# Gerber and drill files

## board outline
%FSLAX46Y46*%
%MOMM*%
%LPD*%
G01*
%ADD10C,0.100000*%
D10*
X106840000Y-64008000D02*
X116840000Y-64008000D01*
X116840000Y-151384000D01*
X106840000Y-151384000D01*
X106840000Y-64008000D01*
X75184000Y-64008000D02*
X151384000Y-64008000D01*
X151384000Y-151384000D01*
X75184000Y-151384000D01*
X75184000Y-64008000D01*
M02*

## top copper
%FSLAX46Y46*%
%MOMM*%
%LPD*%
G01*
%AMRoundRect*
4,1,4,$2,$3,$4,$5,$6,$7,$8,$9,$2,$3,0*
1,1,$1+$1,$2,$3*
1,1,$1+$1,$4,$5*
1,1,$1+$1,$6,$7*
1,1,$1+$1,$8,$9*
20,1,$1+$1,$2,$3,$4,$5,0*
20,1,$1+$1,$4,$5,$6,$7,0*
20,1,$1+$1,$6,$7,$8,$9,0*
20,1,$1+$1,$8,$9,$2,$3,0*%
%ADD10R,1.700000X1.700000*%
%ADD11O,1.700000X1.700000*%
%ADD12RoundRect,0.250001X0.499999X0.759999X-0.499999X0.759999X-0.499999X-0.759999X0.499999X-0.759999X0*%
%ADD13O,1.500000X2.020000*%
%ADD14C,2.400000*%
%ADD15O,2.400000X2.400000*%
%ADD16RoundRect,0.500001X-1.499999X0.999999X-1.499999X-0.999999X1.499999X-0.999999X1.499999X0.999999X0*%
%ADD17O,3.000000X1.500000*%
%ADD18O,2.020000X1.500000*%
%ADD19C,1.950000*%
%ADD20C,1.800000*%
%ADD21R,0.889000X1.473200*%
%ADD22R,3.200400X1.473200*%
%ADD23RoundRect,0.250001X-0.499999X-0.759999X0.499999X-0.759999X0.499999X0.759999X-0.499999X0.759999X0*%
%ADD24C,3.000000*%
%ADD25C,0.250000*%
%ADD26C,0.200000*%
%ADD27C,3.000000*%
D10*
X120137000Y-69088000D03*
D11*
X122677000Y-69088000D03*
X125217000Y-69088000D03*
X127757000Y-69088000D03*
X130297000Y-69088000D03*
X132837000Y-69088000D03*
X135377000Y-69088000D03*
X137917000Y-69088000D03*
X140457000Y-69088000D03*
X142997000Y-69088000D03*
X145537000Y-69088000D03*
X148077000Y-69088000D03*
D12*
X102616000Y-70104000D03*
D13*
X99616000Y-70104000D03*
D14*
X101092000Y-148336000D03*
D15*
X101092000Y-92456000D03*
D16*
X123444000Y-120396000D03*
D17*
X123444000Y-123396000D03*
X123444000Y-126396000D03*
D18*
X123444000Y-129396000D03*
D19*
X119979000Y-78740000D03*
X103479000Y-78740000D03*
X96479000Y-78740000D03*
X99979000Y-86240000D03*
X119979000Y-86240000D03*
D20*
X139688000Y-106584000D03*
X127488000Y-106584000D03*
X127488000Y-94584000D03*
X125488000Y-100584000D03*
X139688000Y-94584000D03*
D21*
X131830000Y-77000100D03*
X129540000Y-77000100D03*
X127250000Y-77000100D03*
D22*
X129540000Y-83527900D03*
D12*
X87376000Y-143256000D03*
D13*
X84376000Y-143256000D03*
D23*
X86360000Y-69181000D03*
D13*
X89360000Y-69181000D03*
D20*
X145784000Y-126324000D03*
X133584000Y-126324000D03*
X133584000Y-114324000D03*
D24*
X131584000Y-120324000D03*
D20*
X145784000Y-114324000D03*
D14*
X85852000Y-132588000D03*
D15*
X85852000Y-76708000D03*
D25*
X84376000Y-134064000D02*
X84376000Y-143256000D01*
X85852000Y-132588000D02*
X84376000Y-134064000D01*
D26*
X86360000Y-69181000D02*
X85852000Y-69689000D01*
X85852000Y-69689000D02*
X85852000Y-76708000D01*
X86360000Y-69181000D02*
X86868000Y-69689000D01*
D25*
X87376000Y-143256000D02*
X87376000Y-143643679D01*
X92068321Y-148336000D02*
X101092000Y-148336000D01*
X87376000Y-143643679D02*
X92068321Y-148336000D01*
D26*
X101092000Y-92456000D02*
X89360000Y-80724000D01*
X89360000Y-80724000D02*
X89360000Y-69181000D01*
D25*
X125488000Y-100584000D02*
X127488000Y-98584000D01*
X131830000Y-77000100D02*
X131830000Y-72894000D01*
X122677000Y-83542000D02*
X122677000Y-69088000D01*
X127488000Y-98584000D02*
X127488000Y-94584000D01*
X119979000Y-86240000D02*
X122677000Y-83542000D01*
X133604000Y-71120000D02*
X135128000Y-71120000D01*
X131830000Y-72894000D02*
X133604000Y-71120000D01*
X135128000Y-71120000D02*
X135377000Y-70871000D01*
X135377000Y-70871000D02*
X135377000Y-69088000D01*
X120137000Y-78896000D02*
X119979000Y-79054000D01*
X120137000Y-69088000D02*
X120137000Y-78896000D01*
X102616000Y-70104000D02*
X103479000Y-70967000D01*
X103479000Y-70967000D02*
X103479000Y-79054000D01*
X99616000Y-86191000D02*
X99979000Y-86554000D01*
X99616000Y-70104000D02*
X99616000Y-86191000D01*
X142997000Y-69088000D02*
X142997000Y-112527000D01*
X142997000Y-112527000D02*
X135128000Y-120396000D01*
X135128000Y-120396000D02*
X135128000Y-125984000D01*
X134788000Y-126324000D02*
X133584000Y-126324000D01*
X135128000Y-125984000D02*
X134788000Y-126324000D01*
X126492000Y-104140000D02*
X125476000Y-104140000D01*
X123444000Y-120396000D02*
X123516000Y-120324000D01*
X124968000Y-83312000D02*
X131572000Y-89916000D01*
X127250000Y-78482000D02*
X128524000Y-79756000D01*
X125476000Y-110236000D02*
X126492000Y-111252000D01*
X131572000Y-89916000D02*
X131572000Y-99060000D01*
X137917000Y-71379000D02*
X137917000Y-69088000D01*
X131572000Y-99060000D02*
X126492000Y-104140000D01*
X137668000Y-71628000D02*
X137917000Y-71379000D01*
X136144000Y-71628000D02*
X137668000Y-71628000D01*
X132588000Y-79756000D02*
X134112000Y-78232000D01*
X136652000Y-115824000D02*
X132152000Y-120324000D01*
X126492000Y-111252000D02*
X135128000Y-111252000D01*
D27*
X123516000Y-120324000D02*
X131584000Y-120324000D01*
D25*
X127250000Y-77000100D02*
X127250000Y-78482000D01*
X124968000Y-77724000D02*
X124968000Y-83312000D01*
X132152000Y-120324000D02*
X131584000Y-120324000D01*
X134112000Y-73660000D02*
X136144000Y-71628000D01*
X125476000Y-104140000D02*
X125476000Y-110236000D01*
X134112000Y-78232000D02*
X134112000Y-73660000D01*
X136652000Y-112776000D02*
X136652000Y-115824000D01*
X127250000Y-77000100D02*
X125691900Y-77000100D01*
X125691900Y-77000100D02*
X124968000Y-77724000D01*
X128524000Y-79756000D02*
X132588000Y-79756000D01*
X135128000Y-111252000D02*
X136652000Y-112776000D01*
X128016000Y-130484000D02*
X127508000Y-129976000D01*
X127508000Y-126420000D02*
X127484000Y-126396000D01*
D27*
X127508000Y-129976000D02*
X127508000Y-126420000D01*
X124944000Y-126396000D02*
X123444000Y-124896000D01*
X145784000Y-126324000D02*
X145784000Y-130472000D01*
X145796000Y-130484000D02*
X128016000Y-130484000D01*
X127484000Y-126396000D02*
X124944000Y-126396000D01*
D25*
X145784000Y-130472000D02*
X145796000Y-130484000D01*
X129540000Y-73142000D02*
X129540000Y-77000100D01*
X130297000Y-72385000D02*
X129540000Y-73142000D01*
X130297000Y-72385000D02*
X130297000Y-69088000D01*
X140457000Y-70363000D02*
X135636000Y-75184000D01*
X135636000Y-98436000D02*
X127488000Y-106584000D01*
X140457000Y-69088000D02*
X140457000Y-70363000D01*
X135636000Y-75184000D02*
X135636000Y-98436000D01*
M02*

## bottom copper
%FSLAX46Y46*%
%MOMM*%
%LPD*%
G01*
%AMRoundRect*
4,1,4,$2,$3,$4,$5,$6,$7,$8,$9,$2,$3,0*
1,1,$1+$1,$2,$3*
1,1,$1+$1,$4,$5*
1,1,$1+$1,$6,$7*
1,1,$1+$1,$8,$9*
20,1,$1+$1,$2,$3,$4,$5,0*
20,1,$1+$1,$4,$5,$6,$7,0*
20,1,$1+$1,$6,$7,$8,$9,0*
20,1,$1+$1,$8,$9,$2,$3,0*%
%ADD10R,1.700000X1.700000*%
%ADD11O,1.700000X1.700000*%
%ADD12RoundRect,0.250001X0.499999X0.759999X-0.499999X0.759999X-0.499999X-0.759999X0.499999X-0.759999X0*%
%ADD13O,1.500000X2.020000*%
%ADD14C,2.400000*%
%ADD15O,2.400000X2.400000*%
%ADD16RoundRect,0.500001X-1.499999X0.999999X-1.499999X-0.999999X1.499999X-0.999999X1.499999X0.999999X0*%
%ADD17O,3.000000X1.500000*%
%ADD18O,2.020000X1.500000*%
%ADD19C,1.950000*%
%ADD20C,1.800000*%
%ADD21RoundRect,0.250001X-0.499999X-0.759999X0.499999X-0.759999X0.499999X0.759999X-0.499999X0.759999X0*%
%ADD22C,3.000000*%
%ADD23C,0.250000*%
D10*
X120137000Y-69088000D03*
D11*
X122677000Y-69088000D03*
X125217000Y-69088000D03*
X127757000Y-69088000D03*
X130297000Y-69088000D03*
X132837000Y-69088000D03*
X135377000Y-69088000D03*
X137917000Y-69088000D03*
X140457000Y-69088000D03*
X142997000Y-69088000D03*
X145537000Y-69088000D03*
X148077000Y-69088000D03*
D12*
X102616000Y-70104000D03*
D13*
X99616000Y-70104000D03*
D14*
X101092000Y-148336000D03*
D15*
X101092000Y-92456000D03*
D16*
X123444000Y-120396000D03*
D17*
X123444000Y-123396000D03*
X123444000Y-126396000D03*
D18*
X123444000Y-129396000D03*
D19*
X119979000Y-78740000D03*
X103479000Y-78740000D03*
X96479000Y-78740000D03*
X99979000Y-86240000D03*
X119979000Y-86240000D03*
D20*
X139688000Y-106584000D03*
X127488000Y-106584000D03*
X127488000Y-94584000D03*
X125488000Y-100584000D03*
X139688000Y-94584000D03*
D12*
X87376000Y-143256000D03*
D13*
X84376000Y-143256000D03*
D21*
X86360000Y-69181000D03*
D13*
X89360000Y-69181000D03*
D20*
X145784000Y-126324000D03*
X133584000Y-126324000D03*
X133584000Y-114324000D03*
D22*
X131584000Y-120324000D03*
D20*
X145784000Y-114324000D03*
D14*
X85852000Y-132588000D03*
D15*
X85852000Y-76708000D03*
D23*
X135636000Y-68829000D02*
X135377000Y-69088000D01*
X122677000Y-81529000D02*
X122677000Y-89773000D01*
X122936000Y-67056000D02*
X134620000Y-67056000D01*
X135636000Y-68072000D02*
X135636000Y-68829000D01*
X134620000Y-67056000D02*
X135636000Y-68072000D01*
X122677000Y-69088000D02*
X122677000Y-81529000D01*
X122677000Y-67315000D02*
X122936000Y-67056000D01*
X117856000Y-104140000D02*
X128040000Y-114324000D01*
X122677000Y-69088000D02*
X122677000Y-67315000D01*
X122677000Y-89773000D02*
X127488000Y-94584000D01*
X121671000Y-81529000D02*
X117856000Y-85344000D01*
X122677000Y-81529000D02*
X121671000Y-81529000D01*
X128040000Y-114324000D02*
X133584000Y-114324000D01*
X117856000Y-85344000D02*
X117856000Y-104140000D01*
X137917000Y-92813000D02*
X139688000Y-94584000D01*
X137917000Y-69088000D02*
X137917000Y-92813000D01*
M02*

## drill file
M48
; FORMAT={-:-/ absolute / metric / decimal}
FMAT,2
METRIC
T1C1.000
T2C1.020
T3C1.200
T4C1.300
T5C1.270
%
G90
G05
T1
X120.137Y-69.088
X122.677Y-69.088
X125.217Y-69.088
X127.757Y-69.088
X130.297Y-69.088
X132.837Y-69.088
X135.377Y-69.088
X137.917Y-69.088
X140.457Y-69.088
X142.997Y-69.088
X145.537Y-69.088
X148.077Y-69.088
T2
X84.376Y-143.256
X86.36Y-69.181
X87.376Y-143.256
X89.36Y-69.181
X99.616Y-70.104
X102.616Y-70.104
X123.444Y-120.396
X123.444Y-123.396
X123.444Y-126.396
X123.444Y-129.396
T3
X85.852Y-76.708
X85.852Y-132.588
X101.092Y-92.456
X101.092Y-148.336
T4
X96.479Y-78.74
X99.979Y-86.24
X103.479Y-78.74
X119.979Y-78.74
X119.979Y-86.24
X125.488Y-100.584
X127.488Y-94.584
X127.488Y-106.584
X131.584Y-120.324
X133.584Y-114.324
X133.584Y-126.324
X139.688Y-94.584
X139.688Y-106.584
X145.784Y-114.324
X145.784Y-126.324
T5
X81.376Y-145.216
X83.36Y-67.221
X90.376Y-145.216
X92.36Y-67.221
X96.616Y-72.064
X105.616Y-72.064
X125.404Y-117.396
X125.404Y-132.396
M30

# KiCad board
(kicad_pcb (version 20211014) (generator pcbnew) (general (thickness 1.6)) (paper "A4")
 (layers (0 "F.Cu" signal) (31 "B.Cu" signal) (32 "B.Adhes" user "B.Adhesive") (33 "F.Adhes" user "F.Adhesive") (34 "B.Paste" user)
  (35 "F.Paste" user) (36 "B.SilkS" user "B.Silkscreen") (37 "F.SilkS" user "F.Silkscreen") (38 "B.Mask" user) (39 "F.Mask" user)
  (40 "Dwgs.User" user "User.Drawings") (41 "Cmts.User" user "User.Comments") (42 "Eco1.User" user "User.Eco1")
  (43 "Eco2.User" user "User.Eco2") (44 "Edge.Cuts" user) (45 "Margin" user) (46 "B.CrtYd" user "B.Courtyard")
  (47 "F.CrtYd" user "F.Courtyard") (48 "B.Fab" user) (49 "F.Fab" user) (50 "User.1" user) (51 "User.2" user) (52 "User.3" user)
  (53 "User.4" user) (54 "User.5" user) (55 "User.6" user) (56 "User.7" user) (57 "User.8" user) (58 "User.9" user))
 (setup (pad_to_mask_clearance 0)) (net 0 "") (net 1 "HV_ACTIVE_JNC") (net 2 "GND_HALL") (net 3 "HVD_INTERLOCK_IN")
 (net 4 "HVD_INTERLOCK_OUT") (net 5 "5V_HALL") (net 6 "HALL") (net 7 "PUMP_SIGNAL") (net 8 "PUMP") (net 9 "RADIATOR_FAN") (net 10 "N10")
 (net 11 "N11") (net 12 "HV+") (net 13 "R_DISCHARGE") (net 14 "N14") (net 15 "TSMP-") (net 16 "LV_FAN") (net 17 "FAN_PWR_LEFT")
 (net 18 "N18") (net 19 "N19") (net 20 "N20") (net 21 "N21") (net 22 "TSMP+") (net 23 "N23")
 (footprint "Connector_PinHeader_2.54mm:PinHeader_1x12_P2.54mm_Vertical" (layer "F.Cu") (at 120.137 69.088 90)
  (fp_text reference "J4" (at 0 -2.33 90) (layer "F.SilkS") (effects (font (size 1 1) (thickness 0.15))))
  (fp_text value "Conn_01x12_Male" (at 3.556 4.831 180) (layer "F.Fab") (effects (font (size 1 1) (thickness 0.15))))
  (pad "1" thru_hole rect (at 0 0 90) (size 1.7 1.7) (drill 1) (layers *.Cu *.Mask) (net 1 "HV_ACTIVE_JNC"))
  (pad "2" thru_hole oval (at 0 2.54 90) (size 1.7 1.7) (drill 1) (layers *.Cu *.Mask) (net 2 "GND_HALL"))
  (pad "3" thru_hole oval (at 0 5.08 90) (size 1.7 1.7) (drill 1) (layers *.Cu *.Mask) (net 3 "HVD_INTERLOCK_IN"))
  (pad "4" thru_hole oval (at 0 7.62 90) (size 1.7 1.7) (drill 1) (layers *.Cu *.Mask) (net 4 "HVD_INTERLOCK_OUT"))
  (pad "5" thru_hole oval (at 0 10.16 90) (size 1.7 1.7) (drill 1) (layers *.Cu *.Mask) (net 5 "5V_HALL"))
  (pad "6" thru_hole oval (at 0 12.7 90) (size 1.7 1.7) (drill 1) (layers *.Cu *.Mask) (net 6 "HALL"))
  (pad "7" thru_hole oval (at 0 15.24 90) (size 1.7 1.7) (drill 1) (layers *.Cu *.Mask) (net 2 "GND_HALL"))
  (pad "8" thru_hole oval (at 0 17.78 90) (size 1.7 1.7) (drill 1) (layers *.Cu *.Mask) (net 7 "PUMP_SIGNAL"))
  (pad "9" thru_hole oval (at 0 20.32 90) (size 1.7 1.7) (drill 1) (layers *.Cu *.Mask) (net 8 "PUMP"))
  (pad "10" thru_hole oval (at 0 22.86 90) (size 1.7 1.7) (drill 1) (layers *.Cu *.Mask) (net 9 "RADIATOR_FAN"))
  (pad "11" thru_hole oval (at 0 25.4 90) (size 1.7 1.7) (drill 1) (layers *.Cu *.Mask) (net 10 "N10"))
  (pad "12" thru_hole oval (at 0 27.94 90) (size 1.7 1.7) (drill 1) (layers *.Cu *.Mask) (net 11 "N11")))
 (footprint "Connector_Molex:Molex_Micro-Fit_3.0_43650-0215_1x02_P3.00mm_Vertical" (layer "F.Cu") (at 102.616 70.104 180)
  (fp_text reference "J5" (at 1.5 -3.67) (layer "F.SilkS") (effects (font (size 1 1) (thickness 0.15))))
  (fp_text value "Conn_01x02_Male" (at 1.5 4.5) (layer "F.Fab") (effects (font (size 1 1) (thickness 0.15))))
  (pad "" np_thru_hole circle (at -3 -1.96 180) (size 1.27 1.27) (drill 1.27) (layers *.Cu *.Mask))
  (pad "" np_thru_hole circle (at 6 -1.96 180) (size 1.27 1.27) (drill 1.27) (layers *.Cu *.Mask))
  (pad "1" thru_hole roundrect (at 0 0 180) (size 1.5 2.02) (drill 1.02) (layers *.Cu *.Mask) (roundrect_rratio 0.166667) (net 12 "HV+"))
  (pad "2" thru_hole oval (at 3 0 180) (size 1.5 2.02) (drill 1.02) (layers *.Cu *.Mask) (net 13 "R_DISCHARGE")))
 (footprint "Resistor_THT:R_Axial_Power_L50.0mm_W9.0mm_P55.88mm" (layer "F.Cu") (at 101.092 148.336 90)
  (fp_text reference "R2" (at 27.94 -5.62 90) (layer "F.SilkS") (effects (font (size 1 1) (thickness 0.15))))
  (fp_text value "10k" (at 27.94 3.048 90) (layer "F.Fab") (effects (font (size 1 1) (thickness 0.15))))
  (pad "1" thru_hole circle (at 0 0 90) (size 2.4 2.4) (drill 1.2) (layers *.Cu *.Mask) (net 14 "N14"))
  (pad "2" thru_hole oval (at 55.88 0 90) (size 2.4 2.4) (drill 1.2) (layers *.Cu *.Mask) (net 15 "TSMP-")))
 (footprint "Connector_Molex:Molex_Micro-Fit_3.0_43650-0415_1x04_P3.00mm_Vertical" (layer "F.Cu") (at 123.444 120.396 -90)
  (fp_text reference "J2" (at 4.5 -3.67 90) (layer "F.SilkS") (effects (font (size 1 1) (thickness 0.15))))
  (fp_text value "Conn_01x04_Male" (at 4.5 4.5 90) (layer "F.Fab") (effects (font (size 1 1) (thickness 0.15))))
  (pad "" np_thru_hole circle (at 12 -1.96 270) (size 1.27 1.27) (drill 1.27) (layers *.Cu *.Mask))
  (pad "" np_thru_hole circle (at -3 -1.96 270) (size 1.27 1.27) (drill 1.27) (layers *.Cu *.Mask))
  (pad "1" thru_hole roundrect (at 0 0 270) (size 3 4) (drill 1.02) (layers *.Cu *.Mask) (roundrect_rratio 0.166667) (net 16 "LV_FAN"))
  (pad "2" thru_hole oval (at 3 0 270) (size 1.5 3) (drill 1.02) (layers *.Cu *.Mask) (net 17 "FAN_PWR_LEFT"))
  (pad "3" thru_hole oval (at 6 0 270) (size 1.5 3) (drill 1.02) (layers *.Cu *.Mask) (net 17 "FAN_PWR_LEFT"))
  (pad "4" thru_hole oval (at 9 0 270) (size 1.5 2.02) (drill 1.02) (layers *.Cu *.Mask) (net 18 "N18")))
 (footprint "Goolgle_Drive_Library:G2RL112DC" (layer "F.Cu") (at 119.979 78.74 180)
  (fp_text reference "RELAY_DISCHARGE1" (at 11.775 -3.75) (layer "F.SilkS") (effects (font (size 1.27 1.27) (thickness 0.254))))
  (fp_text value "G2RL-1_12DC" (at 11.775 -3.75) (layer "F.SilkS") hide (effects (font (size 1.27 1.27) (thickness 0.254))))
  (pad "1" thru_hole circle locked (at 0 0 180) (size 1.95 1.95) (drill 1.3) (layers *.Cu *.Mask) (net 1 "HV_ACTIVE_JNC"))
  (pad "2" thru_hole circle locked (at 16.5 0 180) (size 1.95 1.95) (drill 1.3) (layers *.Cu *.Mask) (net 12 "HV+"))
  (pad "3" thru_hole circle locked (at 23.5 0 180) (size 1.95 1.95) (drill 1.3) (layers *.Cu *.Mask) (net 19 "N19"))
  (pad "4" thru_hole circle locked (at 20 -7.5 180) (size 1.95 1.95) (drill 1.3) (layers *.Cu *.Mask) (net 13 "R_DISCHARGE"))
  (pad "5" thru_hole circle locked (at 0 -7.5 180) (size 1.95 1.95) (drill 1.3) (layers *.Cu *.Mask) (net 2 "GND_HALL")))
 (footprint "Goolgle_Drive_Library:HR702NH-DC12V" (layer "F.Cu") (at 123.088 92.834)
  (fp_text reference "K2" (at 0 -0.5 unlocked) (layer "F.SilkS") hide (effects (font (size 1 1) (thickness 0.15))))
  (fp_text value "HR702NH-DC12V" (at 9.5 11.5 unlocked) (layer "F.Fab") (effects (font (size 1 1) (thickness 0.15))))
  (pad "1" thru_hole circle (at 16.6 13.75) (size 1.8 1.8) (drill 1.3) (layers *.Cu *.Mask) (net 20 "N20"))
  (pad "2" thru_hole circle (at 4.4 13.75) (size 1.8 1.8) (drill 1.3) (layers *.Cu *.Mask) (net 8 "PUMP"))
  (pad "6" thru_hole circle (at 4.4 1.75) (size 1.8 1.8) (drill 1.3) (layers *.Cu *.Mask) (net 2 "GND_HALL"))
  (pad "7" thru_hole circle (at 2.4 7.75) (size 1.8 1.8) (drill 1.3) (layers *.Cu *.Mask) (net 2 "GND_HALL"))
  (pad "14" thru_hole circle (at 16.6 1.75) (size 1.8 1.8) (drill 1.3) (layers *.Cu *.Mask "F.Adhes") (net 7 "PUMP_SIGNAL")))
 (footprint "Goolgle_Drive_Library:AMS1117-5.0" (layer "F.Cu") (at 129.54 80.264 180)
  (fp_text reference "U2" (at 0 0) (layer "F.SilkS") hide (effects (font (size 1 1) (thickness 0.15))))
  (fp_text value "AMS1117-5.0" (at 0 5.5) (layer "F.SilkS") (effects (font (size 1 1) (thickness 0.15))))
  (pad "1" smd rect (at -2.29 3.2639 180) (size 0.889 1.4732) (layers "F.Cu" "F.Paste" "F.Mask") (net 2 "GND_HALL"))
  (pad "2" smd rect (at 0 3.2639 180) (size 0.889 1.4732) (layers "F.Cu" "F.Paste" "F.Mask") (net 5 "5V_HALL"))
  (pad "3" smd rect (at 2.29 3.2639 180) (size 0.889 1.4732) (layers "F.Cu" "F.Paste" "F.Mask") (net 16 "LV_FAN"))
  (pad "4" smd rect (at 0 -3.2639 180) (size 3.2004 1.4732) (layers "F.Cu" "F.Paste" "F.Mask")))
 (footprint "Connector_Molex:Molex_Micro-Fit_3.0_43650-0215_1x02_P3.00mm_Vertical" (layer "F.Cu") (at 87.376 143.256 180)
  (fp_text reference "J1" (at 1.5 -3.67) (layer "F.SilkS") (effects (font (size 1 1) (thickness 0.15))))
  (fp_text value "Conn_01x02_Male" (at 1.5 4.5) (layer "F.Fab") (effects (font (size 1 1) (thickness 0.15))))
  (pad "" np_thru_hole circle (at 6 -1.96 180) (size 1.27 1.27) (drill 1.27) (layers *.Cu *.Mask))
  (pad "" np_thru_hole circle (at -3 -1.96 180) (size 1.27 1.27) (drill 1.27) (layers *.Cu *.Mask))
  (pad "1" thru_hole roundrect (at 0 0 180) (size 1.5 2.02) (drill 1.02) (layers *.Cu *.Mask) (roundrect_rratio 0.166667) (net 14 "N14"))
  (pad "2" thru_hole oval (at 3 0 180) (size 1.5 2.02) (drill 1.02) (layers *.Cu *.Mask) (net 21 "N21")))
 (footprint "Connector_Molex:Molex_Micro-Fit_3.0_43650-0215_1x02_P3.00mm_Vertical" (layer "F.Cu") (at 86.36 69.181)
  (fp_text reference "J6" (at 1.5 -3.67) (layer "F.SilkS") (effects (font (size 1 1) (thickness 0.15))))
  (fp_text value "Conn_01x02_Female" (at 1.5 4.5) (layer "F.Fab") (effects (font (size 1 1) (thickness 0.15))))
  (pad "" np_thru_hole circle (at 6 -1.96) (size 1.27 1.27) (drill 1.27) (layers *.Cu *.Mask))
  (pad "" np_thru_hole circle (at -3 -1.96) (size 1.27 1.27) (drill 1.27) (layers *.Cu *.Mask))
  (pad "1" thru_hole roundrect (at 0 0) (size 1.5 2.02) (drill 1.02) (layers *.Cu *.Mask) (roundrect_rratio 0.166667) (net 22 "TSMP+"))
  (pad "2" thru_hole oval (at 3 0) (size 1.5 2.02) (drill 1.02) (layers *.Cu *.Mask) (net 15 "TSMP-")))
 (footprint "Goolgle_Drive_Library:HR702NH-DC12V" (layer "F.Cu") (at 129.184 112.574)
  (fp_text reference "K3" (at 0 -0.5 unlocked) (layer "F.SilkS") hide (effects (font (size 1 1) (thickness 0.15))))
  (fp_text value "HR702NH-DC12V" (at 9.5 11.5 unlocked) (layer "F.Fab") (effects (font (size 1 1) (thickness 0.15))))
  (pad "1" thru_hole circle (at 16.6 13.75) (size 1.8 1.8) (drill 1.3) (layers *.Cu *.Mask) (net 17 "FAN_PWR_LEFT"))
  (pad "2" thru_hole circle (at 4.4 13.75) (size 1.8 1.8) (drill 1.3) (layers *.Cu *.Mask) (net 9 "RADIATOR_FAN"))
  (pad "6" thru_hole circle (at 4.4 1.75) (size 1.8 1.8) (drill 1.3) (layers *.Cu *.Mask) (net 2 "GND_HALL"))
  (pad "7" thru_hole circle (at 2.4 7.75) (size 3 3) (drill 1.3) (layers *.Cu *.Mask) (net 16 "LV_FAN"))
  (pad "14" thru_hole circle (at 16.6 1.75) (size 1.8 1.8) (drill 1.3) (layers *.Cu *.Mask "F.Adhes") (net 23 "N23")))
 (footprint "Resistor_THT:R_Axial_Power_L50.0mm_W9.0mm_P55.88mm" (layer "F.Cu") (at 85.852 132.588 90)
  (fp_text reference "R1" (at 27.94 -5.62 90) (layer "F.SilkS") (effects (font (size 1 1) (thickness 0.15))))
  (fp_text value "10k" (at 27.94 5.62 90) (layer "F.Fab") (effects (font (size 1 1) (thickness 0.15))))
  (pad "1" thru_hole circle (at 0 0 90) (size 2.4 2.4) (drill 1.2) (layers *.Cu *.Mask) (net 21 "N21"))
  (pad "2" thru_hole oval (at 55.88 0 90) (size 2.4 2.4) (drill 1.2) (layers *.Cu *.Mask) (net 22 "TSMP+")))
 (gr_rect (start 106.84 64.008) (end 116.84 151.384) (layer "Edge.Cuts") (width 0.1) (fill none))
 (gr_rect (start 75.184 64.008) (end 151.384 151.384) (layer "Edge.Cuts") (width 0.1) (fill none))
 (segment (start 84.376 134.064) (end 84.376 143.256) (width 0.25) (layer "F.Cu") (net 21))
 (segment (start 85.852 132.588) (end 84.376 134.064) (width 0.25) (layer "F.Cu") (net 21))
 (segment (start 86.36 69.181) (end 85.852 69.689) (width 0.2) (layer "F.Cu") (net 22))
 (segment (start 85.852 69.689) (end 85.852 76.708) (width 0.2) (layer "F.Cu") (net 22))
 (segment (start 86.36 69.181) (end 86.868 69.689) (width 0.2) (layer "F.Cu") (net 22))
 (segment (start 87.376 143.256) (end 87.376 143.643679) (width 0.25) (layer "F.Cu") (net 14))
 (segment (start 92.068321 148.336) (end 101.092 148.336) (width 0.25) (layer "F.Cu") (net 14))
 (segment (start 87.376 143.643679) (end 92.068321 148.336) (width 0.25) (layer "F.Cu") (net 14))
 (segment (start 101.092 92.456) (end 89.36 80.724) (width 0.2) (layer "F.Cu") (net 15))
 (segment (start 89.36 80.724) (end 89.36 69.181) (width 0.2) (layer "F.Cu") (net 15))
 (segment (start 125.488 100.584) (end 127.488 98.584) (width 0.25) (layer "F.Cu") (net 2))
 (segment (start 131.83 77.0001) (end 131.83 72.894) (width 0.25) (layer "F.Cu") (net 2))
 (segment (start 122.677 83.542) (end 122.677 69.088) (width 0.25) (layer "F.Cu") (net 2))
 (segment (start 127.488 98.584) (end 127.488 94.584) (width 0.25) (layer "F.Cu") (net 2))
 (segment (start 119.979 86.24) (end 122.677 83.542) (width 0.25) (layer "F.Cu") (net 2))
 (segment (start 133.604 71.12) (end 135.128 71.12) (width 0.25) (layer "F.Cu") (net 2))
 (segment (start 131.83 72.894) (end 133.604 71.12) (width 0.25) (layer "F.Cu") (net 2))
 (segment (start 135.128 71.12) (end 135.377 70.871) (width 0.25) (layer "F.Cu") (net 2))
 (segment (start 135.377 70.871) (end 135.377 69.088) (width 0.25) (layer "F.Cu") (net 2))
 (segment (start 135.636 68.829) (end 135.377 69.088) (width 0.25) (layer "B.Cu") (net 2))
 (segment (start 122.677 81.529) (end 122.677 89.773) (width 0.25) (layer "B.Cu") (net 2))
 (segment (start 122.936 67.056) (end 134.62 67.056) (width 0.25) (layer "B.Cu") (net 2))
 (segment (start 135.636 68.072) (end 135.636 68.829) (width 0.25) (layer "B.Cu") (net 2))
 (segment (start 134.62 67.056) (end 135.636 68.072) (width 0.25) (layer "B.Cu") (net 2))
 (segment (start 122.677 69.088) (end 122.677 81.529) (width 0.25) (layer "B.Cu") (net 2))
 (segment (start 122.677 67.315) (end 122.936 67.056) (width 0.25) (layer "B.Cu") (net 2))
 (segment (start 117.856 104.14) (end 128.04 114.324) (width 0.25) (layer "B.Cu") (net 2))
 (segment (start 122.677 69.088) (end 122.677 67.315) (width 0.25) (layer "B.Cu") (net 2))
 (segment (start 122.677 89.773) (end 127.488 94.584) (width 0.25) (layer "B.Cu") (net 2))
 (segment (start 121.671 81.529) (end 117.856 85.344) (width 0.25) (layer "B.Cu") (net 2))
 (segment (start 122.677 81.529) (end 121.671 81.529) (width 0.25) (layer "B.Cu") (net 2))
 (segment (start 128.04 114.324) (end 133.584 114.324) (width 0.25) (layer "B.Cu") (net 2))
 (segment (start 117.856 85.344) (end 117.856 104.14) (width 0.25) (layer "B.Cu") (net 2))
 (segment (start 137.917 92.813) (end 139.688 94.584) (width 0.25) (layer "B.Cu") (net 7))
 (segment (start 137.917 69.088) (end 137.917 92.813) (width 0.25) (layer "B.Cu") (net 7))
 (segment (start 120.137 78.896) (end 119.979 79.054) (width 0.25) (layer "F.Cu") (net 1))
 (segment (start 120.137 69.088) (end 120.137 78.896) (width 0.25) (layer "F.Cu") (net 1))
 (segment (start 102.616 70.104) (end 103.479 70.967) (width 0.25) (layer "F.Cu") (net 12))
 (segment (start 103.479 70.967) (end 103.479 79.054) (width 0.25) (layer "F.Cu") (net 12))
 (segment (start 99.616 86.191) (end 99.979 86.554) (width 0.25) (layer "F.Cu") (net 13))
 (segment (start 99.616 70.104) (end 99.616 86.191) (width 0.25) (layer "F.Cu") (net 13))
 (segment (start 142.997 69.088) (end 142.997 112.527) (width 0.25) (layer "F.Cu") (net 9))
 (segment (start 142.997 112.527) (end 135.128 120.396) (width 0.25) (layer "F.Cu") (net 9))
 (segment (start 135.128 120.396) (end 135.128 125.984) (width 0.25) (layer "F.Cu") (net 9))
 (segment (start 134.788 126.324) (end 133.584 126.324) (width 0.25) (layer "F.Cu") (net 9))
 (segment (start 135.128 125.984) (end 134.788 126.324) (width 0.25) (layer "F.Cu") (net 9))
 (segment (start 126.492 104.14) (end 125.476 104.14) (width 0.25) (layer "F.Cu") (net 16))
 (segment (start 123.444 120.396) (end 123.516 120.324) (width 0.25) (layer "F.Cu") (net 16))
 (segment (start 124.968 83.312) (end 131.572 89.916) (width 0.25) (layer "F.Cu") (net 16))
 (segment (start 127.25 78.482) (end 128.524 79.756) (width 0.25) (layer "F.Cu") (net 16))
 (segment (start 125.476 110.236) (end 126.492 111.252) (width 0.25) (layer "F.Cu") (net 16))
 (segment (start 131.572 89.916) (end 131.572 99.06) (width 0.25) (layer "F.Cu") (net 16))
 (segment (start 137.917 71.379) (end 137.917 69.088) (width 0.25) (layer "F.Cu") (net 16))
 (segment (start 131.572 99.06) (end 126.492 104.14) (width 0.25) (layer "F.Cu") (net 16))
 (segment (start 137.668 71.628) (end 137.917 71.379) (width 0.25) (layer "F.Cu") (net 16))
 (segment (start 136.144 71.628) (end 137.668 71.628) (width 0.25) (layer "F.Cu") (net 16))
 (segment (start 132.588 79.756) (end 134.112 78.232) (width 0.25) (layer "F.Cu") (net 16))
 (segment (start 136.652 115.824) (end 132.152 120.324) (width 0.25) (layer "F.Cu") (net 16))
 (segment (start 126.492 111.252) (end 135.128 111.252) (width 0.25) (layer "F.Cu") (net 16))
 (segment (start 123.516 120.324) (end 131.584 120.324) (width 3) (layer "F.Cu") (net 16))
 (segment (start 127.25 77.0001) (end 127.25 78.482) (width 0.25) (layer "F.Cu") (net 16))
 (segment (start 124.968 77.724) (end 124.968 83.312) (width 0.25) (layer "F.Cu") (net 16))
 (segment (start 132.152 120.324) (end 131.584 120.324) (width 0.25) (layer "F.Cu") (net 16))
 (segment (start 134.112 73.66) (end 136.144 71.628) (width 0.25) (layer "F.Cu") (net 16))
 (segment (start 125.476 104.14) (end 125.476 110.236) (width 0.25) (layer "F.Cu") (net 16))
 (segment (start 134.112 78.232) (end 134.112 73.66) (width 0.25) (layer "F.Cu") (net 16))
 (segment (start 136.652 112.776) (end 136.652 115.824) (width 0.25) (layer "F.Cu") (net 16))
 (segment (start 127.25 77.0001) (end 125.6919 77.0001) (width 0.25) (layer "F.Cu") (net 16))
 (segment (start 125.6919 77.0001) (end 124.968 77.724) (width 0.25) (layer "F.Cu") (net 16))
 (segment (start 128.524 79.756) (end 132.588 79.756) (width 0.25) (layer "F.Cu") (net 16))
 (segment (start 135.128 111.252) (end 136.652 112.776) (width 0.25) (layer "F.Cu") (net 16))
 (segment (start 128.016 130.484) (end 127.508 129.976) (width 0.25) (layer "F.Cu") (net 17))
 (segment (start 127.508 126.42) (end 127.484 126.396) (width 0.25) (layer "F.Cu") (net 17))
 (segment (start 127.508 129.976) (end 127.508 126.42) (width 3) (layer "F.Cu") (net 17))
 (segment (start 124.944 126.396) (end 123.444 124.896) (width 3) (layer "F.Cu") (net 17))
 (segment (start 145.784 126.324) (end 145.784 130.472) (width 3) (layer "F.Cu") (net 17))
 (segment (start 145.796 130.484) (end 128.016 130.484) (width 3) (layer "F.Cu") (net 17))
 (segment (start 127.484 126.396) (end 124.944 126.396) (width 3) (layer "F.Cu") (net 17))
 (segment (start 145.784 130.472) (end 145.796 130.484) (width 0.25) (layer "F.Cu") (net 17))
 (segment (start 129.54 73.142) (end 129.54 77.0001) (width 0.25) (layer "F.Cu") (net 5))
 (segment (start 130.297 72.385) (end 129.54 73.142) (width 0.25) (layer "F.Cu") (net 5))
 (segment (start 130.297 72.385) (end 130.297 69.088) (width 0.25) (layer "F.Cu") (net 5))
 (segment (start 140.457 70.363) (end 135.636 75.184) (width 0.25) (layer "F.Cu") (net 8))
 (segment (start 135.636 98.436) (end 127.488 106.584) (width 0.25) (layer "F.Cu") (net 8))
 (segment (start 140.457 69.088) (end 140.457 70.363) (width 0.25) (layer "F.Cu") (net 8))
 (segment (start 135.636 75.184) (end 135.636 98.436) (width 0.25) (layer "F.Cu") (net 8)))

